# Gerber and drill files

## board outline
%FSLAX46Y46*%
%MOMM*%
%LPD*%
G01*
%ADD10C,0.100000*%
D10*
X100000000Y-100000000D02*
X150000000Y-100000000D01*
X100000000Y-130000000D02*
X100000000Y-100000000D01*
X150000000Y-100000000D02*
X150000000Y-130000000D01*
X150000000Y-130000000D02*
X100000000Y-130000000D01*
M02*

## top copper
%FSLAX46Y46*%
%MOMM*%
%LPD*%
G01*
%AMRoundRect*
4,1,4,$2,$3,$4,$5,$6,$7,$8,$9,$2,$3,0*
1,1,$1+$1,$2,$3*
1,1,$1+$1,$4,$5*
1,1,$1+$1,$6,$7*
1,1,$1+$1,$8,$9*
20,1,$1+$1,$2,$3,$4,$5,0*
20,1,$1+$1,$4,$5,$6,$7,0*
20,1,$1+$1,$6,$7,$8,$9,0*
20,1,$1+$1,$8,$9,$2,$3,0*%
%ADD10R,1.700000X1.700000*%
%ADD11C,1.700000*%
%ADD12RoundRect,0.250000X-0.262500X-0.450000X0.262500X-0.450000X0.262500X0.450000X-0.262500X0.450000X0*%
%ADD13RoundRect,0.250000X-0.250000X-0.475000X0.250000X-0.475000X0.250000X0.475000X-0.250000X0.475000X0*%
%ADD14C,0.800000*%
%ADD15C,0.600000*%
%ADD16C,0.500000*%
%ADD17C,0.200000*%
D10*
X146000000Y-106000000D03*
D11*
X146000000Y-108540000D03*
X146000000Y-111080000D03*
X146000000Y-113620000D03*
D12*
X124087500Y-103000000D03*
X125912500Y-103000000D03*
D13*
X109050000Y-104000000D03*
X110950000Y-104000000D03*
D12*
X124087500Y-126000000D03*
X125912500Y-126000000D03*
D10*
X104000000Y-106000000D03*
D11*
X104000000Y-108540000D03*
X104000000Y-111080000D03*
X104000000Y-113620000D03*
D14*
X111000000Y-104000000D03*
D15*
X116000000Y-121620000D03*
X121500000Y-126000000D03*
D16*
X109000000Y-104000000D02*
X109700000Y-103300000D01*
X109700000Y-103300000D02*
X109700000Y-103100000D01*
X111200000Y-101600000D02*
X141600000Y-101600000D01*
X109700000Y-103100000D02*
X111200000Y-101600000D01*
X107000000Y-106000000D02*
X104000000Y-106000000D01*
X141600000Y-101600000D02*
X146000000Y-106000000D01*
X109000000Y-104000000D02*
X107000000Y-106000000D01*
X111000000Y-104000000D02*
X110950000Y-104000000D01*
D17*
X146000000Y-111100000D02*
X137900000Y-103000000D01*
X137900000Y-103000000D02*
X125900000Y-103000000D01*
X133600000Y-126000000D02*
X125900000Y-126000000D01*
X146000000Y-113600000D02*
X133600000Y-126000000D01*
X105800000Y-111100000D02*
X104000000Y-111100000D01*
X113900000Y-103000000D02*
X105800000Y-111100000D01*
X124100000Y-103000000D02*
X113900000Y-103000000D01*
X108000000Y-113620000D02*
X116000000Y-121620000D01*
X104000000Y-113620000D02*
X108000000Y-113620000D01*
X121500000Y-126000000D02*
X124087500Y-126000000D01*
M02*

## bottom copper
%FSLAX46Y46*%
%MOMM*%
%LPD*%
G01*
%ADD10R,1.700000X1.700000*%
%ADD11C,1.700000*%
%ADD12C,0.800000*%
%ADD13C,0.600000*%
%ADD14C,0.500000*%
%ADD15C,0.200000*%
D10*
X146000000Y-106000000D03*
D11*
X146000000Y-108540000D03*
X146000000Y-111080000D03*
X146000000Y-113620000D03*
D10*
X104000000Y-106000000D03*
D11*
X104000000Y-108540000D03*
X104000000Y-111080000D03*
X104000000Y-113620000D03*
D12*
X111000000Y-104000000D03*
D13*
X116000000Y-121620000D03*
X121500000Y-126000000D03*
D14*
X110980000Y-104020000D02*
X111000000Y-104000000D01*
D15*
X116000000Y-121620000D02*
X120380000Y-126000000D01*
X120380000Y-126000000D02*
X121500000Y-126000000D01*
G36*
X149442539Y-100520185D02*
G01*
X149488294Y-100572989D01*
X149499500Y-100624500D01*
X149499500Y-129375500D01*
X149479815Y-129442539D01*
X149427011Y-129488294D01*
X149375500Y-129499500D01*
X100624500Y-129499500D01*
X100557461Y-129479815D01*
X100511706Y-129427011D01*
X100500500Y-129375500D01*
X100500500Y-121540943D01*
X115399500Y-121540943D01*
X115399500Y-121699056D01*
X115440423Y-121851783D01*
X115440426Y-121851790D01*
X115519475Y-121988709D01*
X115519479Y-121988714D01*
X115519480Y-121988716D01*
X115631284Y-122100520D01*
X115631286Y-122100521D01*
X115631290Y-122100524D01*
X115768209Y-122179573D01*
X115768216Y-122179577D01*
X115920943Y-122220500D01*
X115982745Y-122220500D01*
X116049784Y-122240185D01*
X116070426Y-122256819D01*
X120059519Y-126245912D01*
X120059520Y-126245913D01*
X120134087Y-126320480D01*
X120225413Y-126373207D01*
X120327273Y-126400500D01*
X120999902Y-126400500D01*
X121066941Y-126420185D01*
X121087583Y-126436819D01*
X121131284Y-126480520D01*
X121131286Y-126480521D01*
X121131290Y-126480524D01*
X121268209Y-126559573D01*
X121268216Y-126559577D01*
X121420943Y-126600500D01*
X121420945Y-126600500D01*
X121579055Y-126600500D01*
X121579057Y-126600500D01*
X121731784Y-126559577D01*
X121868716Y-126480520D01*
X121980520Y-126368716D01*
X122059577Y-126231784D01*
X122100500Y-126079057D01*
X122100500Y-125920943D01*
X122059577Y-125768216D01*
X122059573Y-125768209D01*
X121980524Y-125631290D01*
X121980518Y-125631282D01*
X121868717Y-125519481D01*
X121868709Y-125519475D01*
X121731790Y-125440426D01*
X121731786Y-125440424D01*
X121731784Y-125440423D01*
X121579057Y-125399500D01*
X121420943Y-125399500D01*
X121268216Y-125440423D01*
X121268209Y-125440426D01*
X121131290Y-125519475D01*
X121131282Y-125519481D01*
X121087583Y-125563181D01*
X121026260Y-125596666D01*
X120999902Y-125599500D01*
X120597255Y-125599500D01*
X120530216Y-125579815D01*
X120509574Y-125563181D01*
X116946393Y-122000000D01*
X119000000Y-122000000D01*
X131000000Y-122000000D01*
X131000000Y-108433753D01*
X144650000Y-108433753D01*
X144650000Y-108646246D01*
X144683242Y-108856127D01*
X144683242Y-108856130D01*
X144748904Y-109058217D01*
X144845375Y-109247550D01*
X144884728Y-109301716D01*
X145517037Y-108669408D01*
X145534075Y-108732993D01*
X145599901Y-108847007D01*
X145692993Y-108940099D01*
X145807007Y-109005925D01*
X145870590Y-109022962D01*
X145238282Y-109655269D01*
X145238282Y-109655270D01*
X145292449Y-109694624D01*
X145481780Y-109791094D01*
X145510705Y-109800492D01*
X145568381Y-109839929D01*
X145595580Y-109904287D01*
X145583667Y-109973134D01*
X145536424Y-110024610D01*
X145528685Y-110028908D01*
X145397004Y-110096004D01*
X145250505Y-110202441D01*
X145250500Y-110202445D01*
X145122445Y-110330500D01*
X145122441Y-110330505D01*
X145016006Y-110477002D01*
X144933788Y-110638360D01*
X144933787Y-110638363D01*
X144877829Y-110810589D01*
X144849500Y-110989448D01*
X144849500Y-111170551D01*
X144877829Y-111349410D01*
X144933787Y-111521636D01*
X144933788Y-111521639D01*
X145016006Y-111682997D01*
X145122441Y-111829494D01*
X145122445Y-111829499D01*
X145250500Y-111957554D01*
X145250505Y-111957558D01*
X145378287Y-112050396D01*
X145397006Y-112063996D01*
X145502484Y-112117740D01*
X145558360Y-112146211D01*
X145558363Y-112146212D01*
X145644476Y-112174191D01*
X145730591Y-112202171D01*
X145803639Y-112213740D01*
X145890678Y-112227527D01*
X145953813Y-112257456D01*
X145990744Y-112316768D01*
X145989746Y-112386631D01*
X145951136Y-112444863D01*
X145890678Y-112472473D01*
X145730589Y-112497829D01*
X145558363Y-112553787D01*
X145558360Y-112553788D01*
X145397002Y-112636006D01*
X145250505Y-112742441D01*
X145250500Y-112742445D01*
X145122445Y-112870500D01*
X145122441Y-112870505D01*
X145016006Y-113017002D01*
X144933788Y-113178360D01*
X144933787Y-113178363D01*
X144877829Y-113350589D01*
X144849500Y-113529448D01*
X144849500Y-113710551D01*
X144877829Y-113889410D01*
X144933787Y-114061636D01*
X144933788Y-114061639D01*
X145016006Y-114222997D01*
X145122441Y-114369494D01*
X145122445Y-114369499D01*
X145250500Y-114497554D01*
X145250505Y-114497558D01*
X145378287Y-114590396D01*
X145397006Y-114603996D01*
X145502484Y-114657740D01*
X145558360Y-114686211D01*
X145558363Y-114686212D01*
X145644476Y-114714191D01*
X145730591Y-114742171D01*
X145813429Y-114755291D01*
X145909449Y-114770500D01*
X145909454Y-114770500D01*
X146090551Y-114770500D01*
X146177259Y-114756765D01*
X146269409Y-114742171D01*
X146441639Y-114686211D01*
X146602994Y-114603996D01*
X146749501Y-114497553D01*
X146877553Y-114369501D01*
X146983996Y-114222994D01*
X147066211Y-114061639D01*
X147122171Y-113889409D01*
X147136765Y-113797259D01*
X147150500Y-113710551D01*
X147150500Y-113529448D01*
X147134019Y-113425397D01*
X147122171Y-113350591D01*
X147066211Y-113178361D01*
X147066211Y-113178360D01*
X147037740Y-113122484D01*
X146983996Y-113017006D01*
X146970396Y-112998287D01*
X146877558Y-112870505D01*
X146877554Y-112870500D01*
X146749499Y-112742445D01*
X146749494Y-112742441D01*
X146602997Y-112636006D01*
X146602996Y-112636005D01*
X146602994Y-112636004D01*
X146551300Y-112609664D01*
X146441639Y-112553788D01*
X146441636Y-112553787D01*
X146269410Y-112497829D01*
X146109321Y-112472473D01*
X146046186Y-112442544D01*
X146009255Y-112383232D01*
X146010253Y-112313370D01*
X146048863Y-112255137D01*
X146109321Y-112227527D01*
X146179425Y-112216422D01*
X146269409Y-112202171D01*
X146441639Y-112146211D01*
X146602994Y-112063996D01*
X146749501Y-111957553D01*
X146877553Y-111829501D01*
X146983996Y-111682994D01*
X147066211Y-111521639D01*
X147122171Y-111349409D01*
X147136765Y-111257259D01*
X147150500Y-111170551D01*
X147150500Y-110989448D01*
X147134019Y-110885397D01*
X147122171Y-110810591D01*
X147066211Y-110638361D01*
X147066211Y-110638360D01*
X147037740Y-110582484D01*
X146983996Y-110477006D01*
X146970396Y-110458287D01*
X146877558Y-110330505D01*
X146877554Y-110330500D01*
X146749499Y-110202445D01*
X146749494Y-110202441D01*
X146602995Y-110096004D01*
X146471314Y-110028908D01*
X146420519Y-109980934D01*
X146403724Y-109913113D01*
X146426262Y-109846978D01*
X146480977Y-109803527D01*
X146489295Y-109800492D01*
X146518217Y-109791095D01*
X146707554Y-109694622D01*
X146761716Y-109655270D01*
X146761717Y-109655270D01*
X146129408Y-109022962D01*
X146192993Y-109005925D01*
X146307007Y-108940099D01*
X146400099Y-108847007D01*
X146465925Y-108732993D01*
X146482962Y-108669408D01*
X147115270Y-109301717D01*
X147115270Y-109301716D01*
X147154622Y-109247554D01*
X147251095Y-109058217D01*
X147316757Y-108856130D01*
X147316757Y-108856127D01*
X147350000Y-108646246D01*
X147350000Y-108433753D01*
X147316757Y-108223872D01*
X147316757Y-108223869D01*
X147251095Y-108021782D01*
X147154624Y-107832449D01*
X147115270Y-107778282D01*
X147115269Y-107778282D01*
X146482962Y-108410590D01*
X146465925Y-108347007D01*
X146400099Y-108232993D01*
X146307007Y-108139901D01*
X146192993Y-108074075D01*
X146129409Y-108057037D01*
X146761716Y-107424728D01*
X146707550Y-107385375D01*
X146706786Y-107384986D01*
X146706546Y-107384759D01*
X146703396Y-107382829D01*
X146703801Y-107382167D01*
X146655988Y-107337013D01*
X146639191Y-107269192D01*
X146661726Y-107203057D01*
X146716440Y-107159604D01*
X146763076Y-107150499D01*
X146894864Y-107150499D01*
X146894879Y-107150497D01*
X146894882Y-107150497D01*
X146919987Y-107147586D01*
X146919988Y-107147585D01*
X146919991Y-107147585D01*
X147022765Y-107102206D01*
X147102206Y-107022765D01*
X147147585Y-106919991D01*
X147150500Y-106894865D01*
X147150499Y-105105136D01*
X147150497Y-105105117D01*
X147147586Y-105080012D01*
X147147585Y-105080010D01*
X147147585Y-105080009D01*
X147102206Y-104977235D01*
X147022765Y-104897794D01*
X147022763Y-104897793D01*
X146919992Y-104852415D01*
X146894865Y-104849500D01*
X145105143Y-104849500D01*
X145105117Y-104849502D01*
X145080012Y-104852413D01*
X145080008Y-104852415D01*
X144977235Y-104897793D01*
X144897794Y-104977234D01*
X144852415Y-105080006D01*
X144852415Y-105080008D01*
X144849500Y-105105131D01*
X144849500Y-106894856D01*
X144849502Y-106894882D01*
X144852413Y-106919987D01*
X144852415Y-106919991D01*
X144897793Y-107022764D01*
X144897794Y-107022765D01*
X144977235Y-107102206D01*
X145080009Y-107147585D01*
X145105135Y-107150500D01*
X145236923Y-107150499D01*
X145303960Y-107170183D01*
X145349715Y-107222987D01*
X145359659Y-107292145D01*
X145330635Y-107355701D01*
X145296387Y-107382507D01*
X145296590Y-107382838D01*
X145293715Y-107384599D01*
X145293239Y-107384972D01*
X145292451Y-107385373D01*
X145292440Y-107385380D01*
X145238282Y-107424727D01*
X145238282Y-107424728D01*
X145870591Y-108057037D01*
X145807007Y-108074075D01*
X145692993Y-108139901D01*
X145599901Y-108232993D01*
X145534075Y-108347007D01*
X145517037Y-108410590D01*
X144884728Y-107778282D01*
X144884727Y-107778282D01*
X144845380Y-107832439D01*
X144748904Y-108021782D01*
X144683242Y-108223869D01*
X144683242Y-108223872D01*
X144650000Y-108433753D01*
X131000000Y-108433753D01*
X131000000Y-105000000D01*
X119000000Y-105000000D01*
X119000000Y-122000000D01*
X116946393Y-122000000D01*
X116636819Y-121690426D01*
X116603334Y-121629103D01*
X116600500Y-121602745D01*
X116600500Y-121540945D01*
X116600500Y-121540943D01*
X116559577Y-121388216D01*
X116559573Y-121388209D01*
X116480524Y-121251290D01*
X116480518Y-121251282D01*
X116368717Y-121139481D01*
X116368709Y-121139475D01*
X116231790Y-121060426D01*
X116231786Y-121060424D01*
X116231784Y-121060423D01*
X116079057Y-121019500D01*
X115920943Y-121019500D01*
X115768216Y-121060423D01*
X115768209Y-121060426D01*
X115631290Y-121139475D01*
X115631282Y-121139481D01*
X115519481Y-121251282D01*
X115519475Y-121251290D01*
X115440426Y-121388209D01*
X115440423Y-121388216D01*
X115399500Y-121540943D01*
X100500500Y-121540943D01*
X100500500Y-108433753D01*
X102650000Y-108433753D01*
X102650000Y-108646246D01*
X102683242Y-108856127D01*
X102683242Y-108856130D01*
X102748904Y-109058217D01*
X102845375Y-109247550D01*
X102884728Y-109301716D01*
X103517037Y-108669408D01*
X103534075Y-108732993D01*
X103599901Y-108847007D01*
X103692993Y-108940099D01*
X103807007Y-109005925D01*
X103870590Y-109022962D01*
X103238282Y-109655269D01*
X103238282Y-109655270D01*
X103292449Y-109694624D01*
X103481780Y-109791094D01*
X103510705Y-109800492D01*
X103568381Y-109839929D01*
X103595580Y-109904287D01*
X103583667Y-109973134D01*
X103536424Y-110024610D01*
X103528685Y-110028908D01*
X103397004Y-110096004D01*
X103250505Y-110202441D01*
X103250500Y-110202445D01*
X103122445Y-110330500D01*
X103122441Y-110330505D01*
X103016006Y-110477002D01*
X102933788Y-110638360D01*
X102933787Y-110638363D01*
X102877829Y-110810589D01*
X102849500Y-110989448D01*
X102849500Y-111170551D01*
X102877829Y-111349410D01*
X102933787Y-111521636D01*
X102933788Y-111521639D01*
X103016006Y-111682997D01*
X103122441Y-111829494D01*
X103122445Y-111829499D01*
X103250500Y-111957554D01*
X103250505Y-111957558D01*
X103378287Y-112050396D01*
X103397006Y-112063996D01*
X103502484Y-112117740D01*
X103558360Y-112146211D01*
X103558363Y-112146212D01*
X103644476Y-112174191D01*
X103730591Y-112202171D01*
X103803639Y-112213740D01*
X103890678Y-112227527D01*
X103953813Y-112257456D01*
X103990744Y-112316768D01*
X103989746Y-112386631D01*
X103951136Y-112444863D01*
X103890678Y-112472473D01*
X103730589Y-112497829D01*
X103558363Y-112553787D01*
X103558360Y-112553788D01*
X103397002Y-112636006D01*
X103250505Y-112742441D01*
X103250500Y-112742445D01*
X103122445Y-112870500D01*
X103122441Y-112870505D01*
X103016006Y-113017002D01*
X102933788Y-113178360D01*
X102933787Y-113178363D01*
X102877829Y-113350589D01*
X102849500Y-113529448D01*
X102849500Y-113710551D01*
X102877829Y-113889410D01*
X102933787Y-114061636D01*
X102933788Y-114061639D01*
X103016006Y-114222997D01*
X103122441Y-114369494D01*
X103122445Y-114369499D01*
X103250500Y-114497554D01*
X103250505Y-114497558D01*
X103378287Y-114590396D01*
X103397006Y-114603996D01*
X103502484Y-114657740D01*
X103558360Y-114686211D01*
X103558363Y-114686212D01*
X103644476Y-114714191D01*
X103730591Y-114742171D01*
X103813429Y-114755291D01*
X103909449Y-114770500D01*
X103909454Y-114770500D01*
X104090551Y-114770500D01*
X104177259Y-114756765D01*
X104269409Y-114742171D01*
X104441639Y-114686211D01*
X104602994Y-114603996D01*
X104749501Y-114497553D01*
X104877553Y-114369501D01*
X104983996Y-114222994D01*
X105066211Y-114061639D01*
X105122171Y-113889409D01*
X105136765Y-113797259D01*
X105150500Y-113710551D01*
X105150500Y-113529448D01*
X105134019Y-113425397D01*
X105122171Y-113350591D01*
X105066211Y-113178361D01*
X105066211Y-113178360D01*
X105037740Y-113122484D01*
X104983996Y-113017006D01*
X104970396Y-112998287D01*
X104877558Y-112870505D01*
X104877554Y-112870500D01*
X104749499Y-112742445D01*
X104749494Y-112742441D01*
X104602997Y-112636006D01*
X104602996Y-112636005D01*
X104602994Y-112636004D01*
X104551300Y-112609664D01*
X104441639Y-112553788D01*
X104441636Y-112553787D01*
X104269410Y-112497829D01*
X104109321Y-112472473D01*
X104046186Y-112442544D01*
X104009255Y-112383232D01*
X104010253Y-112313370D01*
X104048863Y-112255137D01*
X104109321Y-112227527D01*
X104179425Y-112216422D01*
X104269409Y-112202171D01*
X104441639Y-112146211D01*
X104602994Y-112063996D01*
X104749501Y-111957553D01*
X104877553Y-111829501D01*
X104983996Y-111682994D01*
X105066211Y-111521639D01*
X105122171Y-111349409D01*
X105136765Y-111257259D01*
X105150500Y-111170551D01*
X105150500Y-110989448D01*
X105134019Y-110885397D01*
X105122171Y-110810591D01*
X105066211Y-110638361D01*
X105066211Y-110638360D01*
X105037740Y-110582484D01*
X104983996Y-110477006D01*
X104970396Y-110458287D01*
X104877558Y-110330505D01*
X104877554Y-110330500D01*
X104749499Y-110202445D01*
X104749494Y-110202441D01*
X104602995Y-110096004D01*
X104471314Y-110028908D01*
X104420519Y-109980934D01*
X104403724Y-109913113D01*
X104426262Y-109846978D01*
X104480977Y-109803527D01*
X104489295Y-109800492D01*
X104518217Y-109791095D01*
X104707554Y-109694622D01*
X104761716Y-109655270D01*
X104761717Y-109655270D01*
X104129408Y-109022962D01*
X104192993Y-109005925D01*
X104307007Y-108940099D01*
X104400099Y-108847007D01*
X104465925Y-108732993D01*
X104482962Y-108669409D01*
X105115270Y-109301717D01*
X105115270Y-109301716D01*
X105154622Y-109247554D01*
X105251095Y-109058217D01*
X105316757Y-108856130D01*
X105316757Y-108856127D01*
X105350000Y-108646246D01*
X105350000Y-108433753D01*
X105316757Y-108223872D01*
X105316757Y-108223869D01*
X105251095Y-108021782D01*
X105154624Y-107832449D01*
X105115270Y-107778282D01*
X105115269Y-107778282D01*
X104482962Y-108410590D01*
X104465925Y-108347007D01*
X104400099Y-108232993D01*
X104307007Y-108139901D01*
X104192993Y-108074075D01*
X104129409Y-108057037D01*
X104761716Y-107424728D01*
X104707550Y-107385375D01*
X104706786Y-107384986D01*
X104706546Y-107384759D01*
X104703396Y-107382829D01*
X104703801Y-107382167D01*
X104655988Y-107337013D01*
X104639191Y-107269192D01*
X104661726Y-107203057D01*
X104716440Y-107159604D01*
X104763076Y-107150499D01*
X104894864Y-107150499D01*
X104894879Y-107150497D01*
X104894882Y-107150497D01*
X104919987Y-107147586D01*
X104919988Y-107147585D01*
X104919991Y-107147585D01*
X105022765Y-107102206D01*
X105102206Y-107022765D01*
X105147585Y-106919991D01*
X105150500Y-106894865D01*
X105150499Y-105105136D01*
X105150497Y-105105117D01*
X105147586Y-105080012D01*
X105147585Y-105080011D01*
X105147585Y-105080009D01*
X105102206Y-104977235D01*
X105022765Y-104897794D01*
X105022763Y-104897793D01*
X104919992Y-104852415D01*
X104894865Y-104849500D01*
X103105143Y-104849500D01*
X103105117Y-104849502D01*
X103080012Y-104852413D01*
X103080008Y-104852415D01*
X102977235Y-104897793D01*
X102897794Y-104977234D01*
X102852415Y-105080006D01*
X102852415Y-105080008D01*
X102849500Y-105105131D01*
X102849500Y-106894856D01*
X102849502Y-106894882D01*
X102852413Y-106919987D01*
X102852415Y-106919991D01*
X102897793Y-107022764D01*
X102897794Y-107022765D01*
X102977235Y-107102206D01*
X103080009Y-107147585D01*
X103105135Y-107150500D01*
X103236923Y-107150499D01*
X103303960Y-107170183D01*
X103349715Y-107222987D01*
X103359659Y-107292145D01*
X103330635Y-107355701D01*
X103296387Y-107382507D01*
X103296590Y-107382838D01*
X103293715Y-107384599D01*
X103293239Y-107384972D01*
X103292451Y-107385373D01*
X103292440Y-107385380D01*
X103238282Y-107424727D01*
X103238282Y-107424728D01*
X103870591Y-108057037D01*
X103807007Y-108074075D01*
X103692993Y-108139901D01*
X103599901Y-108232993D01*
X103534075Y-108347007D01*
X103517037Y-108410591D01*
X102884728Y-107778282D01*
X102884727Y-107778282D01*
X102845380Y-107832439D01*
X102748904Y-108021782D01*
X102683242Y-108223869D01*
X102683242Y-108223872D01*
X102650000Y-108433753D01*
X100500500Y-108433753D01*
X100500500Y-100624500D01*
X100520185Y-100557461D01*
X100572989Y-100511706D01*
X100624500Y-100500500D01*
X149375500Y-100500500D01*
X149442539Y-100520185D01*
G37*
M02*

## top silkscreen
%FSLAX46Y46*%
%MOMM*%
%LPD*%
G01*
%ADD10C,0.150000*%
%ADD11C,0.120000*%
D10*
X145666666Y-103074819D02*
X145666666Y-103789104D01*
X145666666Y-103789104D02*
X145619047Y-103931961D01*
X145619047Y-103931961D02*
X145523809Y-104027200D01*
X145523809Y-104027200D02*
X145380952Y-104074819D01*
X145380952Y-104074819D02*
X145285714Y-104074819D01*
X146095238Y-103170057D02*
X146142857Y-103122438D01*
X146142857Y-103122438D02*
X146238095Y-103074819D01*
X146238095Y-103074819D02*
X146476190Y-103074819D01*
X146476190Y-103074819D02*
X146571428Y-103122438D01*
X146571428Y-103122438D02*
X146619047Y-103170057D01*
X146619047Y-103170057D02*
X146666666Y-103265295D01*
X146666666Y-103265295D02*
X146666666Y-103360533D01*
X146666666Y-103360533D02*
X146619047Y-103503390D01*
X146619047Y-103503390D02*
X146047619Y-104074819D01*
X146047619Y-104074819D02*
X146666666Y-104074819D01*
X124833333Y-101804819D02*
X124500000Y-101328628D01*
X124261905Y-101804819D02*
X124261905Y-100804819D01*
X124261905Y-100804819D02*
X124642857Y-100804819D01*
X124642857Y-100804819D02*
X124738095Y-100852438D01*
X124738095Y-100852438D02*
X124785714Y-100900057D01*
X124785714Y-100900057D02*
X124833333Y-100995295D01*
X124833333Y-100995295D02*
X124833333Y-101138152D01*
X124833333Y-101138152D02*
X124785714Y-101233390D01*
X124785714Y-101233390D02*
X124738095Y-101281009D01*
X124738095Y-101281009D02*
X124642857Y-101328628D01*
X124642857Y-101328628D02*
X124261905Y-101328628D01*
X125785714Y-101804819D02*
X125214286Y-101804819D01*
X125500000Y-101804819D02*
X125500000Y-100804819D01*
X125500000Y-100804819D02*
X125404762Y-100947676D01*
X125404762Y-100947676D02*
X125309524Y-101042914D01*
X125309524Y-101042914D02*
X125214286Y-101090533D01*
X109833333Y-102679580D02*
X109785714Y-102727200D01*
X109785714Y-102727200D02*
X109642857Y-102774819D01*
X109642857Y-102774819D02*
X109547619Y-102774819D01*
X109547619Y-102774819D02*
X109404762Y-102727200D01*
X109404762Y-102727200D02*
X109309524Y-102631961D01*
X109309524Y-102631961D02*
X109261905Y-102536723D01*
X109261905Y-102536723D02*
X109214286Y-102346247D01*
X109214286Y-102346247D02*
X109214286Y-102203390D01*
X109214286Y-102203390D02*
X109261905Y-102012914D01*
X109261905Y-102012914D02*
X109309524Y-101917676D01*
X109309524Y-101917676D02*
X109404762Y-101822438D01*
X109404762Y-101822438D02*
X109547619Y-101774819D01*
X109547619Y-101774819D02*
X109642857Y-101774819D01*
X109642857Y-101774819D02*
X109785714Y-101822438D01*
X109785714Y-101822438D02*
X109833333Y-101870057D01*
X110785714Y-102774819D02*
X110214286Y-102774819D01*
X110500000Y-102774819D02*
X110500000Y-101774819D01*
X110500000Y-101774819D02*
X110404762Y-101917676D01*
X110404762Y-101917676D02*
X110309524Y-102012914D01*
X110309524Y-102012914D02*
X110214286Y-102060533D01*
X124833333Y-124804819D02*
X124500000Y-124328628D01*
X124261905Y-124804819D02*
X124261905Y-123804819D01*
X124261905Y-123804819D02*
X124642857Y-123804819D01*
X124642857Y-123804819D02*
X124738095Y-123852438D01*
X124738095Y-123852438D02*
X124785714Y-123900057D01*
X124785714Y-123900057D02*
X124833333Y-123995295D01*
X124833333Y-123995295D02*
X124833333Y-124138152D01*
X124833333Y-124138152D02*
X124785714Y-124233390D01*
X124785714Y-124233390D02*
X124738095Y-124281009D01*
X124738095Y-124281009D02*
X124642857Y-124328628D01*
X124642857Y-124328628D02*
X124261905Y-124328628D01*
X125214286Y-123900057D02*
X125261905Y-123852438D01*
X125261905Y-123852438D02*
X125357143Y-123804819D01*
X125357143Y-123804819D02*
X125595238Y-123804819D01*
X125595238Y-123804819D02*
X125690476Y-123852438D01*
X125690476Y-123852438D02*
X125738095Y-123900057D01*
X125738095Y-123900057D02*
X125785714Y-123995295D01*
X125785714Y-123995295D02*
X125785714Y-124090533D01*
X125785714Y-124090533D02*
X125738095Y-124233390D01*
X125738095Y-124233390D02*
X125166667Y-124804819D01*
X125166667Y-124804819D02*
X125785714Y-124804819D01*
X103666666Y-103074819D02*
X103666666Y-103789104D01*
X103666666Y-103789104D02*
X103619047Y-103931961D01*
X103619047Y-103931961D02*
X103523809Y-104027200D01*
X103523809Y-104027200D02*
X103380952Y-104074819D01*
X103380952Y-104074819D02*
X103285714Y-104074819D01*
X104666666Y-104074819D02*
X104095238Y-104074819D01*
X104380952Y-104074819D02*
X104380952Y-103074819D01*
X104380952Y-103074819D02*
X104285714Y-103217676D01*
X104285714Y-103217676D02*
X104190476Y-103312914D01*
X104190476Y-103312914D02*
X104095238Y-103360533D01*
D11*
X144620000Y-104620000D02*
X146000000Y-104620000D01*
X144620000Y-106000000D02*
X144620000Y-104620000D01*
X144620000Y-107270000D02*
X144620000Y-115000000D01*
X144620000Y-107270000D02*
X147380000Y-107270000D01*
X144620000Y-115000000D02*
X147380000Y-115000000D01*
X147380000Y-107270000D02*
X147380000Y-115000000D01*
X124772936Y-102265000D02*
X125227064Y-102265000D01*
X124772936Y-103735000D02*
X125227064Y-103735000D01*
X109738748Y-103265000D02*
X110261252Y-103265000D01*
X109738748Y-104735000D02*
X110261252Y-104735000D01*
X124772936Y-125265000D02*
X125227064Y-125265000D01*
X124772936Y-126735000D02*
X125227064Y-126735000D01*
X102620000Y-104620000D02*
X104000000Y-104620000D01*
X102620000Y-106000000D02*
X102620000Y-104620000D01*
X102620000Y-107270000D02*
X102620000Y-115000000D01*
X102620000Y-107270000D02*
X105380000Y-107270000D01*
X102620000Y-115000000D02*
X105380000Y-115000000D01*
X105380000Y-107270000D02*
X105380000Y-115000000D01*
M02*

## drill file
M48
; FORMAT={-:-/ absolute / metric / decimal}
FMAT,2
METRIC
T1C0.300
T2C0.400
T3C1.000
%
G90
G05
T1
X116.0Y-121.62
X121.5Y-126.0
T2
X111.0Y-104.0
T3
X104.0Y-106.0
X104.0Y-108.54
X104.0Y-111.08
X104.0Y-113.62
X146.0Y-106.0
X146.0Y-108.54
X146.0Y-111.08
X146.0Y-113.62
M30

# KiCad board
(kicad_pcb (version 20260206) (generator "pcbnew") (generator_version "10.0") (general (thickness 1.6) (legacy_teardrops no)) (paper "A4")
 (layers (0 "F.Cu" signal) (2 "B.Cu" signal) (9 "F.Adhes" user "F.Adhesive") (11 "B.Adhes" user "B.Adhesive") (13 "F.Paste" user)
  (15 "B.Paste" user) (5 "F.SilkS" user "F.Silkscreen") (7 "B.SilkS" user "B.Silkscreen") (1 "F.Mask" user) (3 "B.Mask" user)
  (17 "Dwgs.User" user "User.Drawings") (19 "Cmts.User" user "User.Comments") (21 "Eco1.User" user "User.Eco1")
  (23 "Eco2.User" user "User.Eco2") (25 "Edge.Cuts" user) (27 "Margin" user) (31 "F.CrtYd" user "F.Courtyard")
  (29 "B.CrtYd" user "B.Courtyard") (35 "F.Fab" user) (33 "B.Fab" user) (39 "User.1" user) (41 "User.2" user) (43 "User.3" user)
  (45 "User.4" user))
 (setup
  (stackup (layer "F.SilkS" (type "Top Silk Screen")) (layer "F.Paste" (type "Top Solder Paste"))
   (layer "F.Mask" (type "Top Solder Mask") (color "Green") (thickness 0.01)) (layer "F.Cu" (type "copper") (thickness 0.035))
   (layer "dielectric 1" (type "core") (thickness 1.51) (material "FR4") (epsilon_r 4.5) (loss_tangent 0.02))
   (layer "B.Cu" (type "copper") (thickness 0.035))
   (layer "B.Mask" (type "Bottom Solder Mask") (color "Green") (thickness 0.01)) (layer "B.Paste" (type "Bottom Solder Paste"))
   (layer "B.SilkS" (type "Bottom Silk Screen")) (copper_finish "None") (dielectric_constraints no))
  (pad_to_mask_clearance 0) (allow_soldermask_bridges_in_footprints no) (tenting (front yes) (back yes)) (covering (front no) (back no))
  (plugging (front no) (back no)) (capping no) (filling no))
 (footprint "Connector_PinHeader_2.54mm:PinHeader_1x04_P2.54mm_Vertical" (layer "F.Cu") (at 146 106)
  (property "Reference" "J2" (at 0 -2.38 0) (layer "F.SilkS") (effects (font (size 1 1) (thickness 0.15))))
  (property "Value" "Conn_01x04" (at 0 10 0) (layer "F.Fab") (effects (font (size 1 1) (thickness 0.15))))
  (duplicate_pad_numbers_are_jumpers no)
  (fp_line (start -1.38 -1.38) (end 0 -1.38) (stroke (width 0.12) (type solid)) (layer "F.SilkS"))
  (fp_line (start -1.38 0) (end -1.38 -1.38) (stroke (width 0.12) (type solid)) (layer "F.SilkS"))
  (fp_line (start -1.38 1.27) (end -1.38 9) (stroke (width 0.12) (type solid)) (layer "F.SilkS"))
  (fp_line (start -1.38 1.27) (end 1.38 1.27) (stroke (width 0.12) (type solid)) (layer "F.SilkS"))
  (fp_line (start -1.38 9) (end 1.38 9) (stroke (width 0.12) (type solid)) (layer "F.SilkS"))
  (fp_line (start 1.38 1.27) (end 1.38 9) (stroke (width 0.12) (type solid)) (layer "F.SilkS"))
  (pad "1" thru_hole rect (at 0 0) (size 1.7 1.7) (drill 1) (layers "*.Cu" "*.Mask") (remove_unused_layers no) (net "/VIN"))
  (pad "2" thru_hole circle (at 0 2.54) (size 1.7 1.7) (drill 1) (layers "*.Cu" "*.Mask") (remove_unused_layers no) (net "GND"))
  (pad "3" thru_hole circle (at 0 5.08) (size 1.7 1.7) (drill 1) (layers "*.Cu" "*.Mask") (remove_unused_layers no) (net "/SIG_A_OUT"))
  (pad "4" thru_hole circle (at 0 7.62) (size 1.7 1.7) (drill 1) (layers "*.Cu" "*.Mask") (remove_unused_layers no) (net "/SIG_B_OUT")))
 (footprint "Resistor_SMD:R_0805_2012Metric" (layer "F.Cu") (at 125 103)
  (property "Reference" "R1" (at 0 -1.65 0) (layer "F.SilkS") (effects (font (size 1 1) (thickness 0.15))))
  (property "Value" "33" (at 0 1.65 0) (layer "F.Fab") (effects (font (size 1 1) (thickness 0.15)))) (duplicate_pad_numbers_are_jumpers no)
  (fp_line (start -0.227064 -0.735) (end 0.227064 -0.735) (stroke (width 0.12) (type solid)) (layer "F.SilkS"))
  (fp_line (start -0.227064 0.735) (end 0.227064 0.735) (stroke (width 0.12) (type solid)) (layer "F.SilkS"))
  (pad "1" smd roundrect (at -0.9125 0) (size 1.025 1.4) (layers "F.Cu" "F.Mask" "F.Paste") (roundrect_rratio 0.243902) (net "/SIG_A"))
  (pad "2" smd roundrect (at 0.9125 0) (size 1.025 1.4) (layers "F.Cu" "F.Mask" "F.Paste") (roundrect_rratio 0.243902) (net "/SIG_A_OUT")))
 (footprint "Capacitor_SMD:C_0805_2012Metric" (layer "F.Cu") (at 110 104)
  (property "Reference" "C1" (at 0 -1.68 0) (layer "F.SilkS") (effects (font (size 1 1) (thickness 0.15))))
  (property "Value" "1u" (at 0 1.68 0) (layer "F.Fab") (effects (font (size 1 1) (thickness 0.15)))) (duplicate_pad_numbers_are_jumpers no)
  (fp_line (start -0.261252 -0.735) (end 0.261252 -0.735) (stroke (width 0.12) (type solid)) (layer "F.SilkS"))
  (fp_line (start -0.261252 0.735) (end 0.261252 0.735) (stroke (width 0.12) (type solid)) (layer "F.SilkS"))
  (pad "1" smd roundrect (at -0.95 0) (size 1 1.45) (layers "F.Cu" "F.Mask" "F.Paste") (roundrect_rratio 0.25) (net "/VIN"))
  (pad "2" smd roundrect (at 0.95 0) (size 1 1.45) (layers "F.Cu" "F.Mask" "F.Paste") (roundrect_rratio 0.25) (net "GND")))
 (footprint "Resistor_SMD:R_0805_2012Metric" (layer "F.Cu") (at 125 126)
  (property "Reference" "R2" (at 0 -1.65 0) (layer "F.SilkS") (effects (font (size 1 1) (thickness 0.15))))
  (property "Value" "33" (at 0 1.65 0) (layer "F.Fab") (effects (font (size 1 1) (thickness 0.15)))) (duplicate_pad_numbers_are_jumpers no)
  (fp_line (start -0.227064 -0.735) (end 0.227064 -0.735) (stroke (width 0.12) (type solid)) (layer "F.SilkS"))
  (fp_line (start -0.227064 0.735) (end 0.227064 0.735) (stroke (width 0.12) (type solid)) (layer "F.SilkS"))
  (pad "1" smd roundrect (at -0.9125 0) (size 1.025 1.4) (layers "F.Cu" "F.Mask" "F.Paste") (roundrect_rratio 0.243902) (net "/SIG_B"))
  (pad "2" smd roundrect (at 0.9125 0) (size 1.025 1.4) (layers "F.Cu" "F.Mask" "F.Paste") (roundrect_rratio 0.243902) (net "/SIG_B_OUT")))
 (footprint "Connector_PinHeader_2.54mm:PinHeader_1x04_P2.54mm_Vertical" (layer "F.Cu") (at 104 106)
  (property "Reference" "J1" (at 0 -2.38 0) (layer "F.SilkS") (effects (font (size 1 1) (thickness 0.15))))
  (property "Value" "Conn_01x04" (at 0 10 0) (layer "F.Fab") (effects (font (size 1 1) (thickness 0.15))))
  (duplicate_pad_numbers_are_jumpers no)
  (fp_line (start -1.38 -1.38) (end 0 -1.38) (stroke (width 0.12) (type solid)) (layer "F.SilkS"))
  (fp_line (start -1.38 0) (end -1.38 -1.38) (stroke (width 0.12) (type solid)) (layer "F.SilkS"))
  (fp_line (start -1.38 1.27) (end -1.38 9) (stroke (width 0.12) (type solid)) (layer "F.SilkS"))
  (fp_line (start -1.38 1.27) (end 1.38 1.27) (stroke (width 0.12) (type solid)) (layer "F.SilkS"))
  (fp_line (start -1.38 9) (end 1.38 9) (stroke (width 0.12) (type solid)) (layer "F.SilkS"))
  (fp_line (start 1.38 1.27) (end 1.38 9) (stroke (width 0.12) (type solid)) (layer "F.SilkS"))
  (pad "1" thru_hole rect (at 0 0) (size 1.7 1.7) (drill 1) (layers "*.Cu" "*.Mask") (remove_unused_layers no) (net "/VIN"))
  (pad "2" thru_hole circle (at 0 2.54) (size 1.7 1.7) (drill 1) (layers "*.Cu" "*.Mask") (remove_unused_layers no) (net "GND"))
  (pad "3" thru_hole circle (at 0 5.08) (size 1.7 1.7) (drill 1) (layers "*.Cu" "*.Mask") (remove_unused_layers no) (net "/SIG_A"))
  (pad "4" thru_hole circle (at 0 7.62) (size 1.7 1.7) (drill 1) (layers "*.Cu" "*.Mask") (remove_unused_layers no) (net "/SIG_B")))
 (gr_line (start 100 100) (end 150 100) (stroke (width 0.1) (type default)) (layer "Edge.Cuts"))
 (gr_line (start 100 130) (end 100 100) (stroke (width 0.1) (type default)) (layer "Edge.Cuts"))
 (gr_line (start 150 100) (end 150 130) (stroke (width 0.1) (type default)) (layer "Edge.Cuts"))
 (gr_line (start 150 130) (end 100 130) (stroke (width 0.1) (type default)) (layer "Edge.Cuts"))
 (segment (start 109 104) (end 109.7 103.3) (width 0.5) (layer "F.Cu") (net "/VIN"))
 (segment (start 109.7 103.3) (end 109.7 103.1) (width 0.5) (layer "F.Cu") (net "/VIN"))
 (segment (start 111.2 101.6) (end 141.6 101.6) (width 0.5) (layer "F.Cu") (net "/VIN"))
 (segment (start 109.7 103.1) (end 111.2 101.6) (width 0.5) (layer "F.Cu") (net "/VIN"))
 (segment (start 107 106) (end 104 106) (width 0.5) (layer "F.Cu") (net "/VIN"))
 (segment (start 141.6 101.6) (end 146 106) (width 0.5) (layer "F.Cu") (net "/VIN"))
 (segment (start 109 104) (end 107 106) (width 0.5) (layer "F.Cu") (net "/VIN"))
 (segment (start 111 104) (end 110.95 104) (width 0.5) (layer "F.Cu") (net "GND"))
 (via (at 111 104) (size 0.8) (drill 0.4) (layers "F.Cu" "B.Cu") (capping yes) (filling yes) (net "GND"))
 (segment (start 110.98 104.02) (end 111 104) (width 0.5) (layer "B.Cu") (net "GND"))
 (segment (start 146 111.1) (end 137.9 103) (width 0.2) (layer "F.Cu") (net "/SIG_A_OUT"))
 (segment (start 137.9 103) (end 125.9 103) (width 0.2) (layer "F.Cu") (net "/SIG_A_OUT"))
 (segment (start 133.6 126) (end 125.9 126) (width 0.2) (layer "F.Cu") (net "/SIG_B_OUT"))
 (segment (start 146 113.6) (end 133.6 126) (width 0.2) (layer "F.Cu") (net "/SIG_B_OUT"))
 (segment (start 105.8 111.1) (end 104 111.1) (width 0.2) (layer "F.Cu") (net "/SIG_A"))
 (segment (start 113.9 103) (end 105.8 111.1) (width 0.2) (layer "F.Cu") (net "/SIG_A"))
 (segment (start 124.1 103) (end 113.9 103) (width 0.2) (layer "F.Cu") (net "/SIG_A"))
 (segment (start 108 113.62) (end 116 121.62) (width 0.2) (locked yes) (layer "F.Cu") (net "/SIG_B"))
 (segment (start 104 113.62) (end 108 113.62) (width 0.2) (locked yes) (layer "F.Cu") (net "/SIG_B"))
 (segment (start 121.5 126) (end 124.0875 126) (width 0.2) (locked yes) (layer "F.Cu") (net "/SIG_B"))
 (via (at 116 121.62) (size 0.6) (drill 0.3) (layers "F.Cu" "B.Cu") (locked yes) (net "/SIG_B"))
 (via (at 121.5 126) (size 0.6) (drill 0.3) (layers "F.Cu" "B.Cu") (locked yes) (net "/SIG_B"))
 (segment (start 116 121.62) (end 120.38 126) (width 0.2) (locked yes) (layer "B.Cu") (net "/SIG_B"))
 (segment (start 120.38 126) (end 121.5 126) (width 0.2) (locked yes) (layer "B.Cu") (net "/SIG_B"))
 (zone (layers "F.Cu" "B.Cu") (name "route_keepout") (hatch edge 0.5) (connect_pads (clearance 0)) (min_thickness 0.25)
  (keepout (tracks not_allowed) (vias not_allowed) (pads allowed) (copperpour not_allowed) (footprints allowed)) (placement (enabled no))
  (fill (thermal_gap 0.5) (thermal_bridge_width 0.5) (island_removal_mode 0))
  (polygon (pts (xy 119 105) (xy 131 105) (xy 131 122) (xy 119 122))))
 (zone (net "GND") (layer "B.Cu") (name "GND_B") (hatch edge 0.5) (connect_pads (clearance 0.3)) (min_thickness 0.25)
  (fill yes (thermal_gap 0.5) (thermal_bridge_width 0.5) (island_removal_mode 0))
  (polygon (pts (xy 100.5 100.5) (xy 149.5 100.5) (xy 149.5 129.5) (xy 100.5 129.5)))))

